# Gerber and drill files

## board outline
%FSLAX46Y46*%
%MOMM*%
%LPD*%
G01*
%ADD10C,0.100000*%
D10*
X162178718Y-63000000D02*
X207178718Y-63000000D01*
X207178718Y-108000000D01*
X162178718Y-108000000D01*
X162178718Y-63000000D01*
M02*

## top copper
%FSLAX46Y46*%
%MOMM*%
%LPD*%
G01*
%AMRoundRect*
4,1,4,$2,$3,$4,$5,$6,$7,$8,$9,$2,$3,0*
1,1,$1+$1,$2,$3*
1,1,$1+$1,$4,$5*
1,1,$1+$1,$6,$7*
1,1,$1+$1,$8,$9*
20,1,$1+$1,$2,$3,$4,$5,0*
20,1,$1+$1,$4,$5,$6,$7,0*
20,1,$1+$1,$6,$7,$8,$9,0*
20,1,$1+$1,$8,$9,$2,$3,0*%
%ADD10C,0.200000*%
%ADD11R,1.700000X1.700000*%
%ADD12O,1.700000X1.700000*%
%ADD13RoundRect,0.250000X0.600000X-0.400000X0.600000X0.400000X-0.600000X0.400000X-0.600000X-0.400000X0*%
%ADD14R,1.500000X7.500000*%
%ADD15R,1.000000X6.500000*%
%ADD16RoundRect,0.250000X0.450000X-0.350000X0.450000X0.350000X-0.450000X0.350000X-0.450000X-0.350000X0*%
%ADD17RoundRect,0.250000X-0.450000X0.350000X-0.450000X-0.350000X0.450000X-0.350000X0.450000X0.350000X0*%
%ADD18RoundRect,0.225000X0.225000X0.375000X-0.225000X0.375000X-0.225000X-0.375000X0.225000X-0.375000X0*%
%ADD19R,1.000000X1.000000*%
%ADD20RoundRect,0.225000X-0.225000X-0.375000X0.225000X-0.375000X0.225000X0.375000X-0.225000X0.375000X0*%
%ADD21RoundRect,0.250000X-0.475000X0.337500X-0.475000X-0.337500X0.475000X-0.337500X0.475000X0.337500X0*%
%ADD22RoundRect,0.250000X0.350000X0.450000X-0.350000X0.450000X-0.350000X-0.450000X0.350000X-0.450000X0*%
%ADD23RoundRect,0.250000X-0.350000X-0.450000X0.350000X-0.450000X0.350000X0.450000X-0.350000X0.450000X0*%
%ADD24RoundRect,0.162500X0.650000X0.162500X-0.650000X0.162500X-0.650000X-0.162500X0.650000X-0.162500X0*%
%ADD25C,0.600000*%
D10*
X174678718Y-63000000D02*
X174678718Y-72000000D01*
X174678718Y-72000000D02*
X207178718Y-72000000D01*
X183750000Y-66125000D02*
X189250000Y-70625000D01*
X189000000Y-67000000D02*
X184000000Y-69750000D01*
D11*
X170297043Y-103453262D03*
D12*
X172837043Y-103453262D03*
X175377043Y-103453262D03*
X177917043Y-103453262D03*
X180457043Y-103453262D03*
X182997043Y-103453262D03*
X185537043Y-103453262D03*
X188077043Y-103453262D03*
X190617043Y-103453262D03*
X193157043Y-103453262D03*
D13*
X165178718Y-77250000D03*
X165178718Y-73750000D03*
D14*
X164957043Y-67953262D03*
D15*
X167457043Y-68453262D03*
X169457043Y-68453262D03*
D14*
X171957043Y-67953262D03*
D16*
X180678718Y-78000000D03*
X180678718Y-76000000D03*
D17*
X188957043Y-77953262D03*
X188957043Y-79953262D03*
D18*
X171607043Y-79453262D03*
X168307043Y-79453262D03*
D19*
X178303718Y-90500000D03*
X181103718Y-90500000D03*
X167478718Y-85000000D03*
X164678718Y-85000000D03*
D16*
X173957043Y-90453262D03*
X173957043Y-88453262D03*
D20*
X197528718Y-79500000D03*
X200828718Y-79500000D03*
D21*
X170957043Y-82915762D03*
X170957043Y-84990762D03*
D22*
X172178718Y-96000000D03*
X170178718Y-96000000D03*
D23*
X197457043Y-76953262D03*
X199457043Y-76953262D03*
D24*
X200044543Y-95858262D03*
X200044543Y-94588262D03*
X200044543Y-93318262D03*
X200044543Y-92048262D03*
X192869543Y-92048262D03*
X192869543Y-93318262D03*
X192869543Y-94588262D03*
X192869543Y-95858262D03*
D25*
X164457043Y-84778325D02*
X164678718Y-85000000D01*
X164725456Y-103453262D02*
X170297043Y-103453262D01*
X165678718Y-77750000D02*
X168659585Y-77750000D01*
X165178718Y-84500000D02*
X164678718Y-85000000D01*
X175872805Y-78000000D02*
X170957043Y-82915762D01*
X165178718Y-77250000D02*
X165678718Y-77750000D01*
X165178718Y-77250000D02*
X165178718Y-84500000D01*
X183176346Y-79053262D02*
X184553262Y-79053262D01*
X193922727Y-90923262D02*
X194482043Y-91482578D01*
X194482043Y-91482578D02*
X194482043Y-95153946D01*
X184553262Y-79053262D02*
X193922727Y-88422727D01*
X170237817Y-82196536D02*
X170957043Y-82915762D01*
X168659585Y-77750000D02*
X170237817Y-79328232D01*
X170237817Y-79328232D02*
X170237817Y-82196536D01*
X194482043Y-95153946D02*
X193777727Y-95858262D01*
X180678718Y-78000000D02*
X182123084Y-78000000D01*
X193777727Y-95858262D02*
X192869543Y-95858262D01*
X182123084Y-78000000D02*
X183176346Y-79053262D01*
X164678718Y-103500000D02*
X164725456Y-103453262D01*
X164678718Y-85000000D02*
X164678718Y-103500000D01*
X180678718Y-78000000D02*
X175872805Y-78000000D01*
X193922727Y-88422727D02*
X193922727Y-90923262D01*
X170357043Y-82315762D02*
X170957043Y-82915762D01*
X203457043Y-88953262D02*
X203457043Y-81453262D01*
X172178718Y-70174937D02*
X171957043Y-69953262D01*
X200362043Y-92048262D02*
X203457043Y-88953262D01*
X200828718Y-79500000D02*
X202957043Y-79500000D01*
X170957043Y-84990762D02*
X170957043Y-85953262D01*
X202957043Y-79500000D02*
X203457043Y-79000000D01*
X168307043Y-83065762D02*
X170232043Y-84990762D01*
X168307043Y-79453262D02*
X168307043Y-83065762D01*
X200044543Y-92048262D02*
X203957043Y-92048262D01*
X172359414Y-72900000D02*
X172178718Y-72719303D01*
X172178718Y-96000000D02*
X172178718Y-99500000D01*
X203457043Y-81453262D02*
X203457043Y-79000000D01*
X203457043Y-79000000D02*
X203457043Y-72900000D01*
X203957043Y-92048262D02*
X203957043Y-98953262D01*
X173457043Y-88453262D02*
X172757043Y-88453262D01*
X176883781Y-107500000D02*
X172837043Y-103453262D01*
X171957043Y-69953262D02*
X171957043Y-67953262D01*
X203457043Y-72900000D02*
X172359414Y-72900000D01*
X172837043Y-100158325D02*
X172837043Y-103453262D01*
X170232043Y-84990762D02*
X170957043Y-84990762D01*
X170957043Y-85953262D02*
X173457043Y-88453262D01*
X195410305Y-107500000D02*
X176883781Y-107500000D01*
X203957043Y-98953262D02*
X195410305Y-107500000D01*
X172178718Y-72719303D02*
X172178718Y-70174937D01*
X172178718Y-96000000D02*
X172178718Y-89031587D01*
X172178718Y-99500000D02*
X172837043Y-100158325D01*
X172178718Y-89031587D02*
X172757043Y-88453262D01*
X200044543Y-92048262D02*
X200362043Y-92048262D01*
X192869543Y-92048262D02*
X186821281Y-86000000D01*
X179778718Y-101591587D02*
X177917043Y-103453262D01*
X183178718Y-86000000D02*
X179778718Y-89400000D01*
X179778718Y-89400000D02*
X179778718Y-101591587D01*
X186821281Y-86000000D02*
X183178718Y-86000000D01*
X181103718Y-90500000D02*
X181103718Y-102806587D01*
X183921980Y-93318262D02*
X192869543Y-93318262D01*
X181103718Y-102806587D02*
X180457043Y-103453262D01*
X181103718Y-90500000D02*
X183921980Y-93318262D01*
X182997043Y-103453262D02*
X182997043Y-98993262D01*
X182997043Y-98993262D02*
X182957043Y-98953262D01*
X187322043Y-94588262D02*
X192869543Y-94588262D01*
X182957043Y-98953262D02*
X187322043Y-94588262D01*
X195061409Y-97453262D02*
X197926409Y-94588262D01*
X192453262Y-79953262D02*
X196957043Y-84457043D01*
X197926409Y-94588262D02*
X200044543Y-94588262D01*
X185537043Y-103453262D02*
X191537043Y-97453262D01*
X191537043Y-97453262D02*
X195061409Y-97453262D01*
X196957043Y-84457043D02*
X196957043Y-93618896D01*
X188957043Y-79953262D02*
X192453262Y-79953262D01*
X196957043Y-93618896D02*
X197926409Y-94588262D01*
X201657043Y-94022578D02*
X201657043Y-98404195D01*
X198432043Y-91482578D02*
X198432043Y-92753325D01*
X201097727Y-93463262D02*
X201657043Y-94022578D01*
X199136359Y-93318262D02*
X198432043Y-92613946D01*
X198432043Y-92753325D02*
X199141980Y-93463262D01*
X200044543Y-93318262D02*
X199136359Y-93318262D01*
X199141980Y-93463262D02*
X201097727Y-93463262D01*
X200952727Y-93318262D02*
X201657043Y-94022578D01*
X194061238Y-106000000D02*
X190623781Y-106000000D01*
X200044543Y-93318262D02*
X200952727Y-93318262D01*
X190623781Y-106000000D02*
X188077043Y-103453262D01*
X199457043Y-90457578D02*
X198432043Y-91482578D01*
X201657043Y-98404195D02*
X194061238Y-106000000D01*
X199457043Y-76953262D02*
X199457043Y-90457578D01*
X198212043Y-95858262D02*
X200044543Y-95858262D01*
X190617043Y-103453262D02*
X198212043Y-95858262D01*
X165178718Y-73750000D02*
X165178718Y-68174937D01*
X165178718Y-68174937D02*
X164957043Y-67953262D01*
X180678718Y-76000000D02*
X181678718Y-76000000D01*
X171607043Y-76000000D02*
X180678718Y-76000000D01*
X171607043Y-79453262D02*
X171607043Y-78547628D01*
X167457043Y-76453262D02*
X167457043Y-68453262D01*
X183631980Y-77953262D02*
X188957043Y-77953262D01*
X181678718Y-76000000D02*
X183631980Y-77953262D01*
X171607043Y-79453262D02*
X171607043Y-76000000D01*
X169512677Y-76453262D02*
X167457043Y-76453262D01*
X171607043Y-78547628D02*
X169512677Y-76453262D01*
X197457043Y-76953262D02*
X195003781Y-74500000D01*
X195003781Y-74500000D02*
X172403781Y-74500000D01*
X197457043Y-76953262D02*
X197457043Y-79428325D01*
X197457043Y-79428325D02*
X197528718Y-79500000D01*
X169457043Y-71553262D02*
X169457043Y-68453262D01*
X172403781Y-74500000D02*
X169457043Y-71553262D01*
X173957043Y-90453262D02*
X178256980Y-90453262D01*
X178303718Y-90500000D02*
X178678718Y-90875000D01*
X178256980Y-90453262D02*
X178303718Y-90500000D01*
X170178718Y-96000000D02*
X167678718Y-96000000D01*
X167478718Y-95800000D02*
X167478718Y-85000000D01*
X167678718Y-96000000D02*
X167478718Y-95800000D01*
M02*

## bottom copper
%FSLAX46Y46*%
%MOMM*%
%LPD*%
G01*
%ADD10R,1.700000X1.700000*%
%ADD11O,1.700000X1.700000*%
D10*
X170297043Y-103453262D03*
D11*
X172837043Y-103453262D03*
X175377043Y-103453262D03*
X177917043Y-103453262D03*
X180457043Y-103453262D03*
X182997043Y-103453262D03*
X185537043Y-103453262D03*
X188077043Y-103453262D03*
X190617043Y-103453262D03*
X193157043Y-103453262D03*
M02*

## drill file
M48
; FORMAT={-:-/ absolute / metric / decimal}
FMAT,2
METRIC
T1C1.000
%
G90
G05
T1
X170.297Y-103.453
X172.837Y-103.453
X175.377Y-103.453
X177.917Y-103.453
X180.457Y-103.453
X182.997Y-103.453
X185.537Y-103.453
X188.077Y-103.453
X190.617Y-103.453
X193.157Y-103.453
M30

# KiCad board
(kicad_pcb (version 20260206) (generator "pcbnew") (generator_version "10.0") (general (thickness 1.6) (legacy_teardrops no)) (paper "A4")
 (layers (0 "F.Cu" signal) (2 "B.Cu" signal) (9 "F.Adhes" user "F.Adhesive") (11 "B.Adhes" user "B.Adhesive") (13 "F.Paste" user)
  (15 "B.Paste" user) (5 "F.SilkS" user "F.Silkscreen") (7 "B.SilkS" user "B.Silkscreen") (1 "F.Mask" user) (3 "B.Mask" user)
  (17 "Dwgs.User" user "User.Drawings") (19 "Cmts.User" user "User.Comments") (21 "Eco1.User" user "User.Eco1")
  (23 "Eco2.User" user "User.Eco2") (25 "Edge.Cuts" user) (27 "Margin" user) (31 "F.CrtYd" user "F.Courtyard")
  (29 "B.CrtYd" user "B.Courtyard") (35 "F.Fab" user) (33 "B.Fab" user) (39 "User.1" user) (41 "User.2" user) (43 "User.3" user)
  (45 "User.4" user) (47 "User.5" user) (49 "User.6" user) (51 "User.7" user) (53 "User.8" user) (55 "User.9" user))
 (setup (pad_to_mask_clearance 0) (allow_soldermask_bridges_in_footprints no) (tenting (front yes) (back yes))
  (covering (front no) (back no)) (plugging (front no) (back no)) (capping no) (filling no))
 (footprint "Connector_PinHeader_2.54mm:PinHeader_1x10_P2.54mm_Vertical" (layer "F.Cu") (at 170.297043 103.453262 90)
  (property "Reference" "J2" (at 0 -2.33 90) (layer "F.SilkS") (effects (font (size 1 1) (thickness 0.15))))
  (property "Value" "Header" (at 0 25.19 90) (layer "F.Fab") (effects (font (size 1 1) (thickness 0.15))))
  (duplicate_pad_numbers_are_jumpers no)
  (pad "1" thru_hole rect (at 0 0 90) (size 1.7 1.7) (drill 1) (layers "*.Cu" "*.Mask") (remove_unused_layers no) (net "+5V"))
  (pad "2" thru_hole oval (at 0 2.54 90) (size 1.7 1.7) (drill 1) (layers "*.Cu" "*.Mask") (remove_unused_layers no) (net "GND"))
  (pad "3" thru_hole oval (at 0 5.08 90) (size 1.7 1.7) (drill 1) (layers "*.Cu" "*.Mask") (remove_unused_layers no)
   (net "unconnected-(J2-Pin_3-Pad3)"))
  (pad "4" thru_hole oval (at 0 7.62 90) (size 1.7 1.7) (drill 1) (layers "*.Cu" "*.Mask") (remove_unused_layers no) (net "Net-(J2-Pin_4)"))
  (pad "5" thru_hole oval (at 0 10.16 90) (size 1.7 1.7) (drill 1) (layers "*.Cu" "*.Mask") (remove_unused_layers no) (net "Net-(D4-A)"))
  (pad "6" thru_hole oval (at 0 12.7 90) (size 1.7 1.7) (drill 1) (layers "*.Cu" "*.Mask") (remove_unused_layers no) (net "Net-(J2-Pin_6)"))
  (pad "7" thru_hole oval (at 0 15.24 90) (size 1.7 1.7) (drill 1) (layers "*.Cu" "*.Mask") (remove_unused_layers no) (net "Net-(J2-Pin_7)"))
  (pad "8" thru_hole oval (at 0 17.78 90) (size 1.7 1.7) (drill 1) (layers "*.Cu" "*.Mask") (remove_unused_layers no) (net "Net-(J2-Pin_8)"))
  (pad "9" thru_hole oval (at 0 20.32 90) (size 1.7 1.7) (drill 1) (layers "*.Cu" "*.Mask") (remove_unused_layers no) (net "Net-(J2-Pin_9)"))
  (pad "10" thru_hole oval (at 0 22.86 90) (size 1.7 1.7) (drill 1) (layers "*.Cu" "*.Mask") (remove_unused_layers no)
   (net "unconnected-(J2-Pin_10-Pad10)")))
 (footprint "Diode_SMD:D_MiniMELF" (layer "F.Cu") (at 165.178718 75.5 90)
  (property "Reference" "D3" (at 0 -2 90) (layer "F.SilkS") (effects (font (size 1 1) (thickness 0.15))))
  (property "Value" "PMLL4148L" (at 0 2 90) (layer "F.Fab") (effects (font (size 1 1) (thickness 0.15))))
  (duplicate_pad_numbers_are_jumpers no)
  (pad "1" smd roundrect (at -1.75 0 90) (size 1.3 1.7) (layers "F.Cu" "F.Mask" "F.Paste") (roundrect_rratio 0.1923076923) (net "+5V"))
  (pad "2" smd roundrect (at 1.75 0 90) (size 1.3 1.7) (layers "F.Cu" "F.Mask" "F.Paste") (roundrect_rratio 0.1923076923) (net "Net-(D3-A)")))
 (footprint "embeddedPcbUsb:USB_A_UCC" (layer "F.Cu") (at 168.457043 68.153262 -90)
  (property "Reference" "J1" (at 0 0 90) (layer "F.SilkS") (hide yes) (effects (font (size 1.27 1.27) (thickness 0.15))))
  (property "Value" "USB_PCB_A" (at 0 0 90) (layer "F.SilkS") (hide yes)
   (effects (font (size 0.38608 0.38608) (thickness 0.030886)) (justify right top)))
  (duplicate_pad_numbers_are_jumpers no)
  (pad "1" smd rect (at -0.2 3.5 270) (size 7.5 1.5) (layers "F.Cu" "F.Mask" "F.Paste") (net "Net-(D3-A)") (solder_mask_margin 0.1016))
  (pad "2" smd rect (at 0.3 1 270) (size 6.5 1) (layers "F.Cu" "F.Mask" "F.Paste") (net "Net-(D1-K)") (solder_mask_margin 0.1016))
  (pad "3" smd rect (at 0.3 -1 270) (size 6.5 1) (layers "F.Cu" "F.Mask" "F.Paste") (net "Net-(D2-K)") (solder_mask_margin 0.1016))
  (pad "4" smd rect (at -0.2 -3.5 270) (size 7.5 1.5) (layers "F.Cu" "F.Mask" "F.Paste") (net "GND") (solder_mask_margin 0.1016)))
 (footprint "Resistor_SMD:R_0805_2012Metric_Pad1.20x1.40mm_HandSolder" (layer "F.Cu") (at 180.678718 77 90)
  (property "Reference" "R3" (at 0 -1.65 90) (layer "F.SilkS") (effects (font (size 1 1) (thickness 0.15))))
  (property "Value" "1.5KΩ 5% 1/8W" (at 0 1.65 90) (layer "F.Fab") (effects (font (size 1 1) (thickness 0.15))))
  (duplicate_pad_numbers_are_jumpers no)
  (pad "1" smd roundrect (at -1 0 90) (size 1.2 1.4) (layers "F.Cu" "F.Mask" "F.Paste") (roundrect_rratio 0.208333) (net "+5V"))
  (pad "2" smd roundrect (at 1 0 90) (size 1.2 1.4) (layers "F.Cu" "F.Mask" "F.Paste") (roundrect_rratio 0.208333) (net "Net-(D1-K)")))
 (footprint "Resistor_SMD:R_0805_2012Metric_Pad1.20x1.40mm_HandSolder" (layer "F.Cu") (at 188.957043 78.953262 -90)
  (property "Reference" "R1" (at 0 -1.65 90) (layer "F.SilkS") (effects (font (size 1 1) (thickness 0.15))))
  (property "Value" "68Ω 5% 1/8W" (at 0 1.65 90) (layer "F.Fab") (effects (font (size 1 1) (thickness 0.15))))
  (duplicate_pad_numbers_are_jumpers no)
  (pad "1" smd roundrect (at -1 0 270) (size 1.2 1.4) (layers "F.Cu" "F.Mask" "F.Paste") (roundrect_rratio 0.208333) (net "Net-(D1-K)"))
  (pad "2" smd roundrect (at 1 0 270) (size 1.2 1.4) (layers "F.Cu" "F.Mask" "F.Paste") (roundrect_rratio 0.208333) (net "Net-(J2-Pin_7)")))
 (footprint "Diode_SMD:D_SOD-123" (layer "F.Cu") (at 169.957043 79.453262 180)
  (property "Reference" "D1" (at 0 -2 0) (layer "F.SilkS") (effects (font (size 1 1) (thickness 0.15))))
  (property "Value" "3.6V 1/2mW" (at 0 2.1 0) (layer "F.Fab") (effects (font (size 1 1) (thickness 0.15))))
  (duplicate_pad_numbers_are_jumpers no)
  (pad "1" smd roundrect (at -1.65 0 180) (size 0.9 1.2) (layers "F.Cu" "F.Mask" "F.Paste") (roundrect_rratio 0.25) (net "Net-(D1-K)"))
  (pad "2" smd roundrect (at 1.65 0 180) (size 0.9 1.2) (layers "F.Cu" "F.Mask" "F.Paste") (roundrect_rratio 0.25) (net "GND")))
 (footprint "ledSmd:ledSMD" (layer "F.Cu") (at 180.103718 90.5)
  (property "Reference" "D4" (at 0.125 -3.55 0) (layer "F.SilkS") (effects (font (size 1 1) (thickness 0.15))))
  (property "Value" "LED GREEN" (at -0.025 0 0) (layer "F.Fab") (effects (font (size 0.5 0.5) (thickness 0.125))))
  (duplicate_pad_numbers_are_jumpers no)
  (pad "1" smd rect (at -1.8 0) (size 1 1) (layers "F.Cu" "F.Mask" "F.Paste") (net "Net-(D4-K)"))
  (pad "2" smd rect (at 1 0) (size 1 1) (layers "F.Cu" "F.Mask" "F.Paste") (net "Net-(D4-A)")))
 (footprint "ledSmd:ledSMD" (layer "F.Cu") (at 165.678718 85 180)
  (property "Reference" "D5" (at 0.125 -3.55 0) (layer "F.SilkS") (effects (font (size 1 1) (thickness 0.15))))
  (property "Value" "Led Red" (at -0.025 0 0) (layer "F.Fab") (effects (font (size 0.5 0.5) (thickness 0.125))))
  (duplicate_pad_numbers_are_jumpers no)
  (pad "1" smd rect (at -1.8 0 180) (size 1 1) (layers "F.Cu" "F.Mask" "F.Paste") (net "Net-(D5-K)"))
  (pad "2" smd rect (at 1 0 180) (size 1 1) (layers "F.Cu" "F.Mask" "F.Paste") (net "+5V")))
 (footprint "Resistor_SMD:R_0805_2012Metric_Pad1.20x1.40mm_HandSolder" (layer "F.Cu") (at 173.957043 89.453262 90)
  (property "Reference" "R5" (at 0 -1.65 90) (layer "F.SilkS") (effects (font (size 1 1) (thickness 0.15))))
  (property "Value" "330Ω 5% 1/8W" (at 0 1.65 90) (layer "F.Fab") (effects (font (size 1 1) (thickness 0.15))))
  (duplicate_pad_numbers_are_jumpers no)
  (pad "1" smd roundrect (at -1 0 90) (size 1.2 1.4) (layers "F.Cu" "F.Mask" "F.Paste") (roundrect_rratio 0.208333) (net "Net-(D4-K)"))
  (pad "2" smd roundrect (at 1 0 90) (size 1.2 1.4) (layers "F.Cu" "F.Mask" "F.Paste") (roundrect_rratio 0.208333) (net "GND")))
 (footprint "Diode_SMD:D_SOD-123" (layer "F.Cu") (at 199.178718 79.5)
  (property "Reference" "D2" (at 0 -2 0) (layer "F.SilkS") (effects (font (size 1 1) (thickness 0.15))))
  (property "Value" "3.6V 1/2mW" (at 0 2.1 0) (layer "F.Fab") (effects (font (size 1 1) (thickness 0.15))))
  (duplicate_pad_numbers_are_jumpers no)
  (pad "1" smd roundrect (at -1.65 0) (size 0.9 1.2) (layers "F.Cu" "F.Mask" "F.Paste") (roundrect_rratio 0.25) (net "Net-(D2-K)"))
  (pad "2" smd roundrect (at 1.65 0) (size 0.9 1.2) (layers "F.Cu" "F.Mask" "F.Paste") (roundrect_rratio 0.25) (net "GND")))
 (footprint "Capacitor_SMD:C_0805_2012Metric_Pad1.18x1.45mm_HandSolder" (layer "F.Cu") (at 170.957043 83.953262 -90)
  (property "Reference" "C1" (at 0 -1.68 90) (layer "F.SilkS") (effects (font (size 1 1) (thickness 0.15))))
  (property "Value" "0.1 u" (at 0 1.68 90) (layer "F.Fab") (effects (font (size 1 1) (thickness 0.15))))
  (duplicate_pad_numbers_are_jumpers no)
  (pad "1" smd roundrect (at -1.0375 0 270) (size 1.175 1.45) (layers "F.Cu" "F.Mask" "F.Paste") (roundrect_rratio 0.212766) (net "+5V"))
  (pad "2" smd roundrect (at 1.0375 0 270) (size 1.175 1.45) (layers "F.Cu" "F.Mask" "F.Paste") (roundrect_rratio 0.212766) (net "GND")))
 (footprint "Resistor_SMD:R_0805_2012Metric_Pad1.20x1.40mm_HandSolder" (layer "F.Cu") (at 171.178718 96 180)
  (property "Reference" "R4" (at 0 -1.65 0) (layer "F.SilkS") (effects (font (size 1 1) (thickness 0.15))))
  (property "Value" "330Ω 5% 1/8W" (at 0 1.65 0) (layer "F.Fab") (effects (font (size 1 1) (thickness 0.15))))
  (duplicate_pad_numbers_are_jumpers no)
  (pad "1" smd roundrect (at -1 0 180) (size 1.2 1.4) (layers "F.Cu" "F.Mask" "F.Paste") (roundrect_rratio 0.208333) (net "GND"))
  (pad "2" smd roundrect (at 1 0 180) (size 1.2 1.4) (layers "F.Cu" "F.Mask" "F.Paste") (roundrect_rratio 0.208333) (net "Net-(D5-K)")))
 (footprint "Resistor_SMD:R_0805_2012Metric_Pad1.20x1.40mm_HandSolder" (layer "F.Cu") (at 198.457043 76.953262)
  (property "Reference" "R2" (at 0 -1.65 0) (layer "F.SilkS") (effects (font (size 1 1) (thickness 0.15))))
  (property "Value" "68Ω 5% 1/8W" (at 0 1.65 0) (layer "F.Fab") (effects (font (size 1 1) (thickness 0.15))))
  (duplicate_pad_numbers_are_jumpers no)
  (pad "1" smd roundrect (at -1 0) (size 1.2 1.4) (layers "F.Cu" "F.Mask" "F.Paste") (roundrect_rratio 0.208333) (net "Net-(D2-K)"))
  (pad "2" smd roundrect (at 1 0) (size 1.2 1.4) (layers "F.Cu" "F.Mask" "F.Paste") (roundrect_rratio 0.208333) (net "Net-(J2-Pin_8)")))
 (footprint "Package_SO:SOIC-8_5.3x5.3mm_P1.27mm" (layer "F.Cu") (at 196.457043 93.953262 180)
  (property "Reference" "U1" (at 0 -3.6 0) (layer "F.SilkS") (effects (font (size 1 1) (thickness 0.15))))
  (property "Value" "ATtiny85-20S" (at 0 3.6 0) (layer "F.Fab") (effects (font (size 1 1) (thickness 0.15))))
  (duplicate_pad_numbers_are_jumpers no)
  (pad "1" smd roundrect (at -3.5875 -1.905 180) (size 1.625 0.65) (layers "F.Cu" "F.Mask" "F.Paste") (roundrect_rratio 0.25)
   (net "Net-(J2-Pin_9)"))
  (pad "2" smd roundrect (at -3.5875 -0.635 180) (size 1.625 0.65) (layers "F.Cu" "F.Mask" "F.Paste") (roundrect_rratio 0.25)
   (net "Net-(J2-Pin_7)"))
  (pad "3" smd roundrect (at -3.5875 0.635 180) (size 1.625 0.65) (layers "F.Cu" "F.Mask" "F.Paste") (roundrect_rratio 0.25)
   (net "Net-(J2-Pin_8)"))
  (pad "4" smd roundrect (at -3.5875 1.905 180) (size 1.625 0.65) (layers "F.Cu" "F.Mask" "F.Paste") (roundrect_rratio 0.25) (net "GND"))
  (pad "5" smd roundrect (at 3.5875 1.905 180) (size 1.625 0.65) (layers "F.Cu" "F.Mask" "F.Paste") (roundrect_rratio 0.25)
   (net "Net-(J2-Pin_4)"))
  (pad "6" smd roundrect (at 3.5875 0.635 180) (size 1.625 0.65) (layers "F.Cu" "F.Mask" "F.Paste") (roundrect_rratio 0.25)
   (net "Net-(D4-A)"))
  (pad "7" smd roundrect (at 3.5875 -0.635 180) (size 1.625 0.65) (layers "F.Cu" "F.Mask" "F.Paste") (roundrect_rratio 0.25)
   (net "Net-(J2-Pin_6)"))
  (pad "8" smd roundrect (at 3.5875 -1.905 180) (size 1.625 0.65) (layers "F.Cu" "F.Mask" "F.Paste") (roundrect_rratio 0.25) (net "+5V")))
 (gr_line (start 174.678718 63) (end 174.678718 72) (stroke (width 0.2) (type default)) (layer "F.Cu"))
 (gr_line (start 174.678718 72) (end 207.178718 72) (stroke (width 0.2) (type default)) (layer "F.Cu"))
 (gr_line (start 183.75 66.125) (end 189.25 70.625) (stroke (width 0.2) (type default)) (layer "F.Cu"))
 (gr_line (start 189 67) (end 184 69.75) (stroke (width 0.2) (type default)) (layer "F.Cu"))
 (gr_rect (start 162.178718 63) (end 207.178718 108) (stroke (width 0.1) (type solid)) (fill no) (layer "Edge.Cuts"))
 (segment (start 164.457043 84.778325) (end 164.678718 85) (width 0.6) (layer "F.Cu") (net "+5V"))
 (segment (start 164.725456 103.453262) (end 170.297043 103.453262) (width 0.6) (layer "F.Cu") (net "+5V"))
 (segment (start 165.678718 77.75) (end 168.659585 77.75) (width 0.6) (layer "F.Cu") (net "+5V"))
 (segment (start 165.178718 84.5) (end 164.678718 85) (width 0.6) (layer "F.Cu") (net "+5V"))
 (segment (start 175.872805 78) (end 170.957043 82.915762) (width 0.6) (layer "F.Cu") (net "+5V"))
 (segment (start 165.178718 77.25) (end 165.678718 77.75) (width 0.6) (layer "F.Cu") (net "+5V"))
 (segment (start 165.178718 77.25) (end 165.178718 84.5) (width 0.6) (layer "F.Cu") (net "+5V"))
 (segment (start 183.176346 79.053262) (end 184.553262 79.053262) (width 0.6) (layer "F.Cu") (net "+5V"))
 (segment (start 193.922727 90.923262) (end 194.482043 91.482578) (width 0.6) (layer "F.Cu") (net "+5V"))
 (segment (start 194.482043 91.482578) (end 194.482043 95.153946) (width 0.6) (layer "F.Cu") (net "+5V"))
 (segment (start 184.553262 79.053262) (end 193.922727 88.422727) (width 0.6) (layer "F.Cu") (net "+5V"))
 (segment (start 170.237817 82.196536) (end 170.957043 82.915762) (width 0.6) (layer "F.Cu") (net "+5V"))
 (segment (start 168.659585 77.75) (end 170.237817 79.328232) (width 0.6) (layer "F.Cu") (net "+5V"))
 (segment (start 170.237817 79.328232) (end 170.237817 82.196536) (width 0.6) (layer "F.Cu") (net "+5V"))
 (segment (start 194.482043 95.153946) (end 193.777727 95.858262) (width 0.6) (layer "F.Cu") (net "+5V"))
 (segment (start 180.678718 78) (end 182.123084 78) (width 0.6) (layer "F.Cu") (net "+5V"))
 (segment (start 193.777727 95.858262) (end 192.869543 95.858262) (width 0.6) (layer "F.Cu") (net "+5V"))
 (segment (start 182.123084 78) (end 183.176346 79.053262) (width 0.6) (layer "F.Cu") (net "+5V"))
 (segment (start 164.678718 103.5) (end 164.725456 103.453262) (width 0.6) (layer "F.Cu") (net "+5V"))
 (segment (start 164.678718 85) (end 164.678718 103.5) (width 0.6) (layer "F.Cu") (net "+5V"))
 (segment (start 180.678718 78) (end 175.872805 78) (width 0.6) (layer "F.Cu") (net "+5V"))
 (segment (start 193.922727 88.422727) (end 193.922727 90.923262) (width 0.6) (layer "F.Cu") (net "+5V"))
 (segment (start 170.357043 82.315762) (end 170.957043 82.915762) (width 0.6) (layer "F.Cu") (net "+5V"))
 (segment (start 203.457043 88.953262) (end 203.457043 81.453262) (width 0.6) (layer "F.Cu") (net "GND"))
 (segment (start 172.178718 70.174937) (end 171.957043 69.953262) (width 0.6) (layer "F.Cu") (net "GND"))
 (segment (start 200.362043 92.048262) (end 203.457043 88.953262) (width 0.6) (layer "F.Cu") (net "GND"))
 (segment (start 200.828718 79.5) (end 202.957043 79.5) (width 0.6) (layer "F.Cu") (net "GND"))
 (segment (start 170.957043 84.990762) (end 170.957043 85.953262) (width 0.6) (layer "F.Cu") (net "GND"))
 (segment (start 202.957043 79.5) (end 203.457043 79) (width 0.6) (layer "F.Cu") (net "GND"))
 (segment (start 168.307043 83.065762) (end 170.232043 84.990762) (width 0.6) (layer "F.Cu") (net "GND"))
 (segment (start 168.307043 79.453262) (end 168.307043 83.065762) (width 0.6) (layer "F.Cu") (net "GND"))
 (segment (start 200.044543 92.048262) (end 203.957043 92.048262) (width 0.6) (layer "F.Cu") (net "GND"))
 (segment (start 172.359414 72.9) (end 172.178718 72.719303) (width 0.6) (layer "F.Cu") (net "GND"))
 (segment (start 172.178718 96) (end 172.178718 99.5) (width 0.6) (layer "F.Cu") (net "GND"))
 (segment (start 203.457043 81.453262) (end 203.457043 79) (width 0.6) (layer "F.Cu") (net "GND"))
 (segment (start 203.457043 79) (end 203.457043 72.9) (width 0.6) (layer "F.Cu") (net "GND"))
 (segment (start 203.957043 92.048262) (end 203.957043 98.953262) (width 0.6) (layer "F.Cu") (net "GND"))
 (segment (start 173.457043 88.453262) (end 172.757043 88.453262) (width 0.6) (layer "F.Cu") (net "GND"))
 (segment (start 176.883781 107.5) (end 172.837043 103.453262) (width 0.6) (layer "F.Cu") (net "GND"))
 (segment (start 171.957043 69.953262) (end 171.957043 67.953262) (width 0.6) (layer "F.Cu") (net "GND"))
 (segment (start 203.457043 72.9) (end 172.359414 72.9) (width 0.6) (layer "F.Cu") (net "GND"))
 (segment (start 172.837043 100.158325) (end 172.837043 103.453262) (width 0.6) (layer "F.Cu") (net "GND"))
 (segment (start 170.232043 84.990762) (end 170.957043 84.990762) (width 0.6) (layer "F.Cu") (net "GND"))
 (segment (start 170.957043 85.953262) (end 173.457043 88.453262) (width 0.6) (layer "F.Cu") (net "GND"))
 (segment (start 195.410305 107.5) (end 176.883781 107.5) (width 0.6) (layer "F.Cu") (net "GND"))
 (segment (start 203.957043 98.953262) (end 195.410305 107.5) (width 0.6) (layer "F.Cu") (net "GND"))
 (segment (start 172.178718 72.719303) (end 172.178718 70.174937) (width 0.6) (layer "F.Cu") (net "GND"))
 (segment (start 172.178718 96) (end 172.178718 89.031587) (width 0.6) (layer "F.Cu") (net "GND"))
 (segment (start 172.178718 99.5) (end 172.837043 100.158325) (width 0.6) (layer "F.Cu") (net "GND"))
 (segment (start 172.178718 89.031587) (end 172.757043 88.453262) (width 0.6) (layer "F.Cu") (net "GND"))
 (segment (start 200.044543 92.048262) (end 200.362043 92.048262) (width 0.6) (layer "F.Cu") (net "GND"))
 (segment (start 192.869543 92.048262) (end 186.821281 86) (width 0.6) (layer "F.Cu") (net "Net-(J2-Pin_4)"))
 (segment (start 179.778718 101.591587) (end 177.917043 103.453262) (width 0.6) (layer "F.Cu") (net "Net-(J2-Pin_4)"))
 (segment (start 183.178718 86) (end 179.778718 89.4) (width 0.6) (layer "F.Cu") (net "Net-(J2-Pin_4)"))
 (segment (start 179.778718 89.4) (end 179.778718 101.591587) (width 0.6) (layer "F.Cu") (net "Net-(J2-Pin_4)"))
 (segment (start 186.821281 86) (end 183.178718 86) (width 0.6) (layer "F.Cu") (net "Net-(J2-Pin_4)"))
 (segment (start 181.103718 90.5) (end 181.103718 102.806587) (width 0.6) (layer "F.Cu") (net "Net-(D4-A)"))
 (segment (start 183.92198 93.318262) (end 192.869543 93.318262) (width 0.6) (layer "F.Cu") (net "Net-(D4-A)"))
 (segment (start 181.103718 102.806587) (end 180.457043 103.453262) (width 0.6) (layer "F.Cu") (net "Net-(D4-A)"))
 (segment (start 181.103718 90.5) (end 183.92198 93.318262) (width 0.6) (layer "F.Cu") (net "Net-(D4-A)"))
 (segment (start 182.997043 103.453262) (end 182.997043 98.993262) (width 0.6) (layer "F.Cu") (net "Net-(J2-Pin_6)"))
 (segment (start 182.997043 98.993262) (end 182.957043 98.953262) (width 0.6) (layer "F.Cu") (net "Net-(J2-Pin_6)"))
 (segment (start 187.322043 94.588262) (end 192.869543 94.588262) (width 0.6) (layer "F.Cu") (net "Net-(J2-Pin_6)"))
 (segment (start 182.957043 98.953262) (end 187.322043 94.588262) (width 0.6) (layer "F.Cu") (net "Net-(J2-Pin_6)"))
 (segment (start 195.061409 97.453262) (end 197.926409 94.588262) (width 0.6) (layer "F.Cu") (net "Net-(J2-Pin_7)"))
 (segment (start 192.453262 79.953262) (end 196.957043 84.457043) (width 0.6) (layer "F.Cu") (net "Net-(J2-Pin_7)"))
 (segment (start 197.926409 94.588262) (end 200.044543 94.588262) (width 0.6) (layer "F.Cu") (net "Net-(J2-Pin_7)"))
 (segment (start 185.537043 103.453262) (end 191.537043 97.453262) (width 0.6) (layer "F.Cu") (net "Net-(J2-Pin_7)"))
 (segment (start 191.537043 97.453262) (end 195.061409 97.453262) (width 0.6) (layer "F.Cu") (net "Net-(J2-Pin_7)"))
 (segment (start 196.957043 84.457043) (end 196.957043 93.618896) (width 0.6) (layer "F.Cu") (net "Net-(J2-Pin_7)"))
 (segment (start 188.957043 79.953262) (end 192.453262 79.953262) (width 0.6) (layer "F.Cu") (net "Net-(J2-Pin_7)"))
 (segment (start 196.957043 93.618896) (end 197.926409 94.588262) (width 0.6) (layer "F.Cu") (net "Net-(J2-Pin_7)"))
 (segment (start 201.657043 94.022578) (end 201.657043 98.404195) (width 0.6) (layer "F.Cu") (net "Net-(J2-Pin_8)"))
 (segment (start 198.432043 91.482578) (end 198.432043 92.753325) (width 0.6) (layer "F.Cu") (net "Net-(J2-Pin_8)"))
 (segment (start 201.097727 93.463262) (end 201.657043 94.022578) (width 0.6) (layer "F.Cu") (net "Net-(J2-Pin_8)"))
 (segment (start 199.136359 93.318262) (end 198.432043 92.613946) (width 0.6) (layer "F.Cu") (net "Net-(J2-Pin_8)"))
 (segment (start 198.432043 92.753325) (end 199.14198 93.463262) (width 0.6) (layer "F.Cu") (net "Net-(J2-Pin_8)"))
 (segment (start 200.044543 93.318262) (end 199.136359 93.318262) (width 0.6) (layer "F.Cu") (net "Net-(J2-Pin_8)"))
 (segment (start 199.14198 93.463262) (end 201.097727 93.463262) (width 0.6) (layer "F.Cu") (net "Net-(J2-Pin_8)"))
 (segment (start 200.952727 93.318262) (end 201.657043 94.022578) (width 0.6) (layer "F.Cu") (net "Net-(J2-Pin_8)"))
 (segment (start 194.061238 106) (end 190.623781 106) (width 0.6) (layer "F.Cu") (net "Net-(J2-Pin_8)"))
 (segment (start 200.044543 93.318262) (end 200.952727 93.318262) (width 0.6) (layer "F.Cu") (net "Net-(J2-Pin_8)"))
 (segment (start 190.623781 106) (end 188.077043 103.453262) (width 0.6) (layer "F.Cu") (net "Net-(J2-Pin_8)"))
 (segment (start 199.457043 90.457578) (end 198.432043 91.482578) (width 0.6) (layer "F.Cu") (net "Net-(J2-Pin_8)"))
 (segment (start 201.657043 98.404195) (end 194.061238 106) (width 0.6) (layer "F.Cu") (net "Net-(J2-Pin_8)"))
 (segment (start 199.457043 76.953262) (end 199.457043 90.457578) (width 0.6) (layer "F.Cu") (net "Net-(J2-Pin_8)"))
 (segment (start 198.212043 95.858262) (end 200.044543 95.858262) (width 0.6) (layer "F.Cu") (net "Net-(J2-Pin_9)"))
 (segment (start 190.617043 103.453262) (end 198.212043 95.858262) (width 0.6) (layer "F.Cu") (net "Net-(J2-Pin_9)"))
 (segment (start 165.178718 73.75) (end 165.178718 68.174937) (width 0.6) (layer "F.Cu") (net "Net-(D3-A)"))
 (segment (start 165.178718 68.174937) (end 164.957043 67.953262) (width 0.6) (layer "F.Cu") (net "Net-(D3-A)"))
 (segment (start 180.678718 76) (end 181.678718 76) (width 0.6) (layer "F.Cu") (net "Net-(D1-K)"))
 (segment (start 171.607043 76) (end 180.678718 76) (width 0.6) (layer "F.Cu") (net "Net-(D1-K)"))
 (segment (start 171.607043 79.453262) (end 171.607043 78.547628) (width 0.6) (layer "F.Cu") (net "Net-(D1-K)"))
 (segment (start 167.457043 76.453262) (end 167.457043 68.453262) (width 0.6) (layer "F.Cu") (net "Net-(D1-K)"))
 (segment (start 183.63198 77.953262) (end 188.957043 77.953262) (width 0.6) (layer "F.Cu") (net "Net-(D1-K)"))
 (segment (start 181.678718 76) (end 183.63198 77.953262) (width 0.6) (layer "F.Cu") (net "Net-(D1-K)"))
 (segment (start 171.607043 79.453262) (end 171.607043 76) (width 0.6) (layer "F.Cu") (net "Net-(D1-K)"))
 (segment (start 169.512677 76.453262) (end 167.457043 76.453262) (width 0.6) (layer "F.Cu") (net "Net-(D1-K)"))
 (segment (start 171.607043 78.547628) (end 169.512677 76.453262) (width 0.6) (layer "F.Cu") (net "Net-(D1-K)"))
 (segment (start 197.457043 76.953262) (end 195.003781 74.5) (width 0.6) (layer "F.Cu") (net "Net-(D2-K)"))
 (segment (start 195.003781 74.5) (end 172.403781 74.5) (width 0.6) (layer "F.Cu") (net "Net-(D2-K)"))
 (segment (start 197.457043 76.953262) (end 197.457043 79.428325) (width 0.6) (layer "F.Cu") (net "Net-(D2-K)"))
 (segment (start 197.457043 79.428325) (end 197.528718 79.5) (width 0.6) (layer "F.Cu") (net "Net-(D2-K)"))
 (segment (start 169.457043 71.553262) (end 169.457043 68.453262) (width 0.6) (layer "F.Cu") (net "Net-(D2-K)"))
 (segment (start 172.403781 74.5) (end 169.457043 71.553262) (width 0.6) (layer "F.Cu") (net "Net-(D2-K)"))
 (segment (start 173.957043 90.453262) (end 178.25698 90.453262) (width 0.6) (layer "F.Cu") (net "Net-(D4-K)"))
 (segment (start 178.303718 90.5) (end 178.678718 90.875) (width 0.6) (layer "F.Cu") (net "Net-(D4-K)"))
 (segment (start 178.25698 90.453262) (end 178.303718 90.5) (width 0.6) (layer "F.Cu") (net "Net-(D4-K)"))
 (segment (start 170.178718 96) (end 167.678718 96) (width 0.6) (layer "F.Cu") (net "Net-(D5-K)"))
 (segment (start 167.478718 95.8) (end 167.478718 85) (width 0.6) (layer "F.Cu") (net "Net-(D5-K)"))
 (segment (start 167.678718 96) (end 167.478718 95.8) (width 0.6) (layer "F.Cu") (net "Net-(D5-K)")))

